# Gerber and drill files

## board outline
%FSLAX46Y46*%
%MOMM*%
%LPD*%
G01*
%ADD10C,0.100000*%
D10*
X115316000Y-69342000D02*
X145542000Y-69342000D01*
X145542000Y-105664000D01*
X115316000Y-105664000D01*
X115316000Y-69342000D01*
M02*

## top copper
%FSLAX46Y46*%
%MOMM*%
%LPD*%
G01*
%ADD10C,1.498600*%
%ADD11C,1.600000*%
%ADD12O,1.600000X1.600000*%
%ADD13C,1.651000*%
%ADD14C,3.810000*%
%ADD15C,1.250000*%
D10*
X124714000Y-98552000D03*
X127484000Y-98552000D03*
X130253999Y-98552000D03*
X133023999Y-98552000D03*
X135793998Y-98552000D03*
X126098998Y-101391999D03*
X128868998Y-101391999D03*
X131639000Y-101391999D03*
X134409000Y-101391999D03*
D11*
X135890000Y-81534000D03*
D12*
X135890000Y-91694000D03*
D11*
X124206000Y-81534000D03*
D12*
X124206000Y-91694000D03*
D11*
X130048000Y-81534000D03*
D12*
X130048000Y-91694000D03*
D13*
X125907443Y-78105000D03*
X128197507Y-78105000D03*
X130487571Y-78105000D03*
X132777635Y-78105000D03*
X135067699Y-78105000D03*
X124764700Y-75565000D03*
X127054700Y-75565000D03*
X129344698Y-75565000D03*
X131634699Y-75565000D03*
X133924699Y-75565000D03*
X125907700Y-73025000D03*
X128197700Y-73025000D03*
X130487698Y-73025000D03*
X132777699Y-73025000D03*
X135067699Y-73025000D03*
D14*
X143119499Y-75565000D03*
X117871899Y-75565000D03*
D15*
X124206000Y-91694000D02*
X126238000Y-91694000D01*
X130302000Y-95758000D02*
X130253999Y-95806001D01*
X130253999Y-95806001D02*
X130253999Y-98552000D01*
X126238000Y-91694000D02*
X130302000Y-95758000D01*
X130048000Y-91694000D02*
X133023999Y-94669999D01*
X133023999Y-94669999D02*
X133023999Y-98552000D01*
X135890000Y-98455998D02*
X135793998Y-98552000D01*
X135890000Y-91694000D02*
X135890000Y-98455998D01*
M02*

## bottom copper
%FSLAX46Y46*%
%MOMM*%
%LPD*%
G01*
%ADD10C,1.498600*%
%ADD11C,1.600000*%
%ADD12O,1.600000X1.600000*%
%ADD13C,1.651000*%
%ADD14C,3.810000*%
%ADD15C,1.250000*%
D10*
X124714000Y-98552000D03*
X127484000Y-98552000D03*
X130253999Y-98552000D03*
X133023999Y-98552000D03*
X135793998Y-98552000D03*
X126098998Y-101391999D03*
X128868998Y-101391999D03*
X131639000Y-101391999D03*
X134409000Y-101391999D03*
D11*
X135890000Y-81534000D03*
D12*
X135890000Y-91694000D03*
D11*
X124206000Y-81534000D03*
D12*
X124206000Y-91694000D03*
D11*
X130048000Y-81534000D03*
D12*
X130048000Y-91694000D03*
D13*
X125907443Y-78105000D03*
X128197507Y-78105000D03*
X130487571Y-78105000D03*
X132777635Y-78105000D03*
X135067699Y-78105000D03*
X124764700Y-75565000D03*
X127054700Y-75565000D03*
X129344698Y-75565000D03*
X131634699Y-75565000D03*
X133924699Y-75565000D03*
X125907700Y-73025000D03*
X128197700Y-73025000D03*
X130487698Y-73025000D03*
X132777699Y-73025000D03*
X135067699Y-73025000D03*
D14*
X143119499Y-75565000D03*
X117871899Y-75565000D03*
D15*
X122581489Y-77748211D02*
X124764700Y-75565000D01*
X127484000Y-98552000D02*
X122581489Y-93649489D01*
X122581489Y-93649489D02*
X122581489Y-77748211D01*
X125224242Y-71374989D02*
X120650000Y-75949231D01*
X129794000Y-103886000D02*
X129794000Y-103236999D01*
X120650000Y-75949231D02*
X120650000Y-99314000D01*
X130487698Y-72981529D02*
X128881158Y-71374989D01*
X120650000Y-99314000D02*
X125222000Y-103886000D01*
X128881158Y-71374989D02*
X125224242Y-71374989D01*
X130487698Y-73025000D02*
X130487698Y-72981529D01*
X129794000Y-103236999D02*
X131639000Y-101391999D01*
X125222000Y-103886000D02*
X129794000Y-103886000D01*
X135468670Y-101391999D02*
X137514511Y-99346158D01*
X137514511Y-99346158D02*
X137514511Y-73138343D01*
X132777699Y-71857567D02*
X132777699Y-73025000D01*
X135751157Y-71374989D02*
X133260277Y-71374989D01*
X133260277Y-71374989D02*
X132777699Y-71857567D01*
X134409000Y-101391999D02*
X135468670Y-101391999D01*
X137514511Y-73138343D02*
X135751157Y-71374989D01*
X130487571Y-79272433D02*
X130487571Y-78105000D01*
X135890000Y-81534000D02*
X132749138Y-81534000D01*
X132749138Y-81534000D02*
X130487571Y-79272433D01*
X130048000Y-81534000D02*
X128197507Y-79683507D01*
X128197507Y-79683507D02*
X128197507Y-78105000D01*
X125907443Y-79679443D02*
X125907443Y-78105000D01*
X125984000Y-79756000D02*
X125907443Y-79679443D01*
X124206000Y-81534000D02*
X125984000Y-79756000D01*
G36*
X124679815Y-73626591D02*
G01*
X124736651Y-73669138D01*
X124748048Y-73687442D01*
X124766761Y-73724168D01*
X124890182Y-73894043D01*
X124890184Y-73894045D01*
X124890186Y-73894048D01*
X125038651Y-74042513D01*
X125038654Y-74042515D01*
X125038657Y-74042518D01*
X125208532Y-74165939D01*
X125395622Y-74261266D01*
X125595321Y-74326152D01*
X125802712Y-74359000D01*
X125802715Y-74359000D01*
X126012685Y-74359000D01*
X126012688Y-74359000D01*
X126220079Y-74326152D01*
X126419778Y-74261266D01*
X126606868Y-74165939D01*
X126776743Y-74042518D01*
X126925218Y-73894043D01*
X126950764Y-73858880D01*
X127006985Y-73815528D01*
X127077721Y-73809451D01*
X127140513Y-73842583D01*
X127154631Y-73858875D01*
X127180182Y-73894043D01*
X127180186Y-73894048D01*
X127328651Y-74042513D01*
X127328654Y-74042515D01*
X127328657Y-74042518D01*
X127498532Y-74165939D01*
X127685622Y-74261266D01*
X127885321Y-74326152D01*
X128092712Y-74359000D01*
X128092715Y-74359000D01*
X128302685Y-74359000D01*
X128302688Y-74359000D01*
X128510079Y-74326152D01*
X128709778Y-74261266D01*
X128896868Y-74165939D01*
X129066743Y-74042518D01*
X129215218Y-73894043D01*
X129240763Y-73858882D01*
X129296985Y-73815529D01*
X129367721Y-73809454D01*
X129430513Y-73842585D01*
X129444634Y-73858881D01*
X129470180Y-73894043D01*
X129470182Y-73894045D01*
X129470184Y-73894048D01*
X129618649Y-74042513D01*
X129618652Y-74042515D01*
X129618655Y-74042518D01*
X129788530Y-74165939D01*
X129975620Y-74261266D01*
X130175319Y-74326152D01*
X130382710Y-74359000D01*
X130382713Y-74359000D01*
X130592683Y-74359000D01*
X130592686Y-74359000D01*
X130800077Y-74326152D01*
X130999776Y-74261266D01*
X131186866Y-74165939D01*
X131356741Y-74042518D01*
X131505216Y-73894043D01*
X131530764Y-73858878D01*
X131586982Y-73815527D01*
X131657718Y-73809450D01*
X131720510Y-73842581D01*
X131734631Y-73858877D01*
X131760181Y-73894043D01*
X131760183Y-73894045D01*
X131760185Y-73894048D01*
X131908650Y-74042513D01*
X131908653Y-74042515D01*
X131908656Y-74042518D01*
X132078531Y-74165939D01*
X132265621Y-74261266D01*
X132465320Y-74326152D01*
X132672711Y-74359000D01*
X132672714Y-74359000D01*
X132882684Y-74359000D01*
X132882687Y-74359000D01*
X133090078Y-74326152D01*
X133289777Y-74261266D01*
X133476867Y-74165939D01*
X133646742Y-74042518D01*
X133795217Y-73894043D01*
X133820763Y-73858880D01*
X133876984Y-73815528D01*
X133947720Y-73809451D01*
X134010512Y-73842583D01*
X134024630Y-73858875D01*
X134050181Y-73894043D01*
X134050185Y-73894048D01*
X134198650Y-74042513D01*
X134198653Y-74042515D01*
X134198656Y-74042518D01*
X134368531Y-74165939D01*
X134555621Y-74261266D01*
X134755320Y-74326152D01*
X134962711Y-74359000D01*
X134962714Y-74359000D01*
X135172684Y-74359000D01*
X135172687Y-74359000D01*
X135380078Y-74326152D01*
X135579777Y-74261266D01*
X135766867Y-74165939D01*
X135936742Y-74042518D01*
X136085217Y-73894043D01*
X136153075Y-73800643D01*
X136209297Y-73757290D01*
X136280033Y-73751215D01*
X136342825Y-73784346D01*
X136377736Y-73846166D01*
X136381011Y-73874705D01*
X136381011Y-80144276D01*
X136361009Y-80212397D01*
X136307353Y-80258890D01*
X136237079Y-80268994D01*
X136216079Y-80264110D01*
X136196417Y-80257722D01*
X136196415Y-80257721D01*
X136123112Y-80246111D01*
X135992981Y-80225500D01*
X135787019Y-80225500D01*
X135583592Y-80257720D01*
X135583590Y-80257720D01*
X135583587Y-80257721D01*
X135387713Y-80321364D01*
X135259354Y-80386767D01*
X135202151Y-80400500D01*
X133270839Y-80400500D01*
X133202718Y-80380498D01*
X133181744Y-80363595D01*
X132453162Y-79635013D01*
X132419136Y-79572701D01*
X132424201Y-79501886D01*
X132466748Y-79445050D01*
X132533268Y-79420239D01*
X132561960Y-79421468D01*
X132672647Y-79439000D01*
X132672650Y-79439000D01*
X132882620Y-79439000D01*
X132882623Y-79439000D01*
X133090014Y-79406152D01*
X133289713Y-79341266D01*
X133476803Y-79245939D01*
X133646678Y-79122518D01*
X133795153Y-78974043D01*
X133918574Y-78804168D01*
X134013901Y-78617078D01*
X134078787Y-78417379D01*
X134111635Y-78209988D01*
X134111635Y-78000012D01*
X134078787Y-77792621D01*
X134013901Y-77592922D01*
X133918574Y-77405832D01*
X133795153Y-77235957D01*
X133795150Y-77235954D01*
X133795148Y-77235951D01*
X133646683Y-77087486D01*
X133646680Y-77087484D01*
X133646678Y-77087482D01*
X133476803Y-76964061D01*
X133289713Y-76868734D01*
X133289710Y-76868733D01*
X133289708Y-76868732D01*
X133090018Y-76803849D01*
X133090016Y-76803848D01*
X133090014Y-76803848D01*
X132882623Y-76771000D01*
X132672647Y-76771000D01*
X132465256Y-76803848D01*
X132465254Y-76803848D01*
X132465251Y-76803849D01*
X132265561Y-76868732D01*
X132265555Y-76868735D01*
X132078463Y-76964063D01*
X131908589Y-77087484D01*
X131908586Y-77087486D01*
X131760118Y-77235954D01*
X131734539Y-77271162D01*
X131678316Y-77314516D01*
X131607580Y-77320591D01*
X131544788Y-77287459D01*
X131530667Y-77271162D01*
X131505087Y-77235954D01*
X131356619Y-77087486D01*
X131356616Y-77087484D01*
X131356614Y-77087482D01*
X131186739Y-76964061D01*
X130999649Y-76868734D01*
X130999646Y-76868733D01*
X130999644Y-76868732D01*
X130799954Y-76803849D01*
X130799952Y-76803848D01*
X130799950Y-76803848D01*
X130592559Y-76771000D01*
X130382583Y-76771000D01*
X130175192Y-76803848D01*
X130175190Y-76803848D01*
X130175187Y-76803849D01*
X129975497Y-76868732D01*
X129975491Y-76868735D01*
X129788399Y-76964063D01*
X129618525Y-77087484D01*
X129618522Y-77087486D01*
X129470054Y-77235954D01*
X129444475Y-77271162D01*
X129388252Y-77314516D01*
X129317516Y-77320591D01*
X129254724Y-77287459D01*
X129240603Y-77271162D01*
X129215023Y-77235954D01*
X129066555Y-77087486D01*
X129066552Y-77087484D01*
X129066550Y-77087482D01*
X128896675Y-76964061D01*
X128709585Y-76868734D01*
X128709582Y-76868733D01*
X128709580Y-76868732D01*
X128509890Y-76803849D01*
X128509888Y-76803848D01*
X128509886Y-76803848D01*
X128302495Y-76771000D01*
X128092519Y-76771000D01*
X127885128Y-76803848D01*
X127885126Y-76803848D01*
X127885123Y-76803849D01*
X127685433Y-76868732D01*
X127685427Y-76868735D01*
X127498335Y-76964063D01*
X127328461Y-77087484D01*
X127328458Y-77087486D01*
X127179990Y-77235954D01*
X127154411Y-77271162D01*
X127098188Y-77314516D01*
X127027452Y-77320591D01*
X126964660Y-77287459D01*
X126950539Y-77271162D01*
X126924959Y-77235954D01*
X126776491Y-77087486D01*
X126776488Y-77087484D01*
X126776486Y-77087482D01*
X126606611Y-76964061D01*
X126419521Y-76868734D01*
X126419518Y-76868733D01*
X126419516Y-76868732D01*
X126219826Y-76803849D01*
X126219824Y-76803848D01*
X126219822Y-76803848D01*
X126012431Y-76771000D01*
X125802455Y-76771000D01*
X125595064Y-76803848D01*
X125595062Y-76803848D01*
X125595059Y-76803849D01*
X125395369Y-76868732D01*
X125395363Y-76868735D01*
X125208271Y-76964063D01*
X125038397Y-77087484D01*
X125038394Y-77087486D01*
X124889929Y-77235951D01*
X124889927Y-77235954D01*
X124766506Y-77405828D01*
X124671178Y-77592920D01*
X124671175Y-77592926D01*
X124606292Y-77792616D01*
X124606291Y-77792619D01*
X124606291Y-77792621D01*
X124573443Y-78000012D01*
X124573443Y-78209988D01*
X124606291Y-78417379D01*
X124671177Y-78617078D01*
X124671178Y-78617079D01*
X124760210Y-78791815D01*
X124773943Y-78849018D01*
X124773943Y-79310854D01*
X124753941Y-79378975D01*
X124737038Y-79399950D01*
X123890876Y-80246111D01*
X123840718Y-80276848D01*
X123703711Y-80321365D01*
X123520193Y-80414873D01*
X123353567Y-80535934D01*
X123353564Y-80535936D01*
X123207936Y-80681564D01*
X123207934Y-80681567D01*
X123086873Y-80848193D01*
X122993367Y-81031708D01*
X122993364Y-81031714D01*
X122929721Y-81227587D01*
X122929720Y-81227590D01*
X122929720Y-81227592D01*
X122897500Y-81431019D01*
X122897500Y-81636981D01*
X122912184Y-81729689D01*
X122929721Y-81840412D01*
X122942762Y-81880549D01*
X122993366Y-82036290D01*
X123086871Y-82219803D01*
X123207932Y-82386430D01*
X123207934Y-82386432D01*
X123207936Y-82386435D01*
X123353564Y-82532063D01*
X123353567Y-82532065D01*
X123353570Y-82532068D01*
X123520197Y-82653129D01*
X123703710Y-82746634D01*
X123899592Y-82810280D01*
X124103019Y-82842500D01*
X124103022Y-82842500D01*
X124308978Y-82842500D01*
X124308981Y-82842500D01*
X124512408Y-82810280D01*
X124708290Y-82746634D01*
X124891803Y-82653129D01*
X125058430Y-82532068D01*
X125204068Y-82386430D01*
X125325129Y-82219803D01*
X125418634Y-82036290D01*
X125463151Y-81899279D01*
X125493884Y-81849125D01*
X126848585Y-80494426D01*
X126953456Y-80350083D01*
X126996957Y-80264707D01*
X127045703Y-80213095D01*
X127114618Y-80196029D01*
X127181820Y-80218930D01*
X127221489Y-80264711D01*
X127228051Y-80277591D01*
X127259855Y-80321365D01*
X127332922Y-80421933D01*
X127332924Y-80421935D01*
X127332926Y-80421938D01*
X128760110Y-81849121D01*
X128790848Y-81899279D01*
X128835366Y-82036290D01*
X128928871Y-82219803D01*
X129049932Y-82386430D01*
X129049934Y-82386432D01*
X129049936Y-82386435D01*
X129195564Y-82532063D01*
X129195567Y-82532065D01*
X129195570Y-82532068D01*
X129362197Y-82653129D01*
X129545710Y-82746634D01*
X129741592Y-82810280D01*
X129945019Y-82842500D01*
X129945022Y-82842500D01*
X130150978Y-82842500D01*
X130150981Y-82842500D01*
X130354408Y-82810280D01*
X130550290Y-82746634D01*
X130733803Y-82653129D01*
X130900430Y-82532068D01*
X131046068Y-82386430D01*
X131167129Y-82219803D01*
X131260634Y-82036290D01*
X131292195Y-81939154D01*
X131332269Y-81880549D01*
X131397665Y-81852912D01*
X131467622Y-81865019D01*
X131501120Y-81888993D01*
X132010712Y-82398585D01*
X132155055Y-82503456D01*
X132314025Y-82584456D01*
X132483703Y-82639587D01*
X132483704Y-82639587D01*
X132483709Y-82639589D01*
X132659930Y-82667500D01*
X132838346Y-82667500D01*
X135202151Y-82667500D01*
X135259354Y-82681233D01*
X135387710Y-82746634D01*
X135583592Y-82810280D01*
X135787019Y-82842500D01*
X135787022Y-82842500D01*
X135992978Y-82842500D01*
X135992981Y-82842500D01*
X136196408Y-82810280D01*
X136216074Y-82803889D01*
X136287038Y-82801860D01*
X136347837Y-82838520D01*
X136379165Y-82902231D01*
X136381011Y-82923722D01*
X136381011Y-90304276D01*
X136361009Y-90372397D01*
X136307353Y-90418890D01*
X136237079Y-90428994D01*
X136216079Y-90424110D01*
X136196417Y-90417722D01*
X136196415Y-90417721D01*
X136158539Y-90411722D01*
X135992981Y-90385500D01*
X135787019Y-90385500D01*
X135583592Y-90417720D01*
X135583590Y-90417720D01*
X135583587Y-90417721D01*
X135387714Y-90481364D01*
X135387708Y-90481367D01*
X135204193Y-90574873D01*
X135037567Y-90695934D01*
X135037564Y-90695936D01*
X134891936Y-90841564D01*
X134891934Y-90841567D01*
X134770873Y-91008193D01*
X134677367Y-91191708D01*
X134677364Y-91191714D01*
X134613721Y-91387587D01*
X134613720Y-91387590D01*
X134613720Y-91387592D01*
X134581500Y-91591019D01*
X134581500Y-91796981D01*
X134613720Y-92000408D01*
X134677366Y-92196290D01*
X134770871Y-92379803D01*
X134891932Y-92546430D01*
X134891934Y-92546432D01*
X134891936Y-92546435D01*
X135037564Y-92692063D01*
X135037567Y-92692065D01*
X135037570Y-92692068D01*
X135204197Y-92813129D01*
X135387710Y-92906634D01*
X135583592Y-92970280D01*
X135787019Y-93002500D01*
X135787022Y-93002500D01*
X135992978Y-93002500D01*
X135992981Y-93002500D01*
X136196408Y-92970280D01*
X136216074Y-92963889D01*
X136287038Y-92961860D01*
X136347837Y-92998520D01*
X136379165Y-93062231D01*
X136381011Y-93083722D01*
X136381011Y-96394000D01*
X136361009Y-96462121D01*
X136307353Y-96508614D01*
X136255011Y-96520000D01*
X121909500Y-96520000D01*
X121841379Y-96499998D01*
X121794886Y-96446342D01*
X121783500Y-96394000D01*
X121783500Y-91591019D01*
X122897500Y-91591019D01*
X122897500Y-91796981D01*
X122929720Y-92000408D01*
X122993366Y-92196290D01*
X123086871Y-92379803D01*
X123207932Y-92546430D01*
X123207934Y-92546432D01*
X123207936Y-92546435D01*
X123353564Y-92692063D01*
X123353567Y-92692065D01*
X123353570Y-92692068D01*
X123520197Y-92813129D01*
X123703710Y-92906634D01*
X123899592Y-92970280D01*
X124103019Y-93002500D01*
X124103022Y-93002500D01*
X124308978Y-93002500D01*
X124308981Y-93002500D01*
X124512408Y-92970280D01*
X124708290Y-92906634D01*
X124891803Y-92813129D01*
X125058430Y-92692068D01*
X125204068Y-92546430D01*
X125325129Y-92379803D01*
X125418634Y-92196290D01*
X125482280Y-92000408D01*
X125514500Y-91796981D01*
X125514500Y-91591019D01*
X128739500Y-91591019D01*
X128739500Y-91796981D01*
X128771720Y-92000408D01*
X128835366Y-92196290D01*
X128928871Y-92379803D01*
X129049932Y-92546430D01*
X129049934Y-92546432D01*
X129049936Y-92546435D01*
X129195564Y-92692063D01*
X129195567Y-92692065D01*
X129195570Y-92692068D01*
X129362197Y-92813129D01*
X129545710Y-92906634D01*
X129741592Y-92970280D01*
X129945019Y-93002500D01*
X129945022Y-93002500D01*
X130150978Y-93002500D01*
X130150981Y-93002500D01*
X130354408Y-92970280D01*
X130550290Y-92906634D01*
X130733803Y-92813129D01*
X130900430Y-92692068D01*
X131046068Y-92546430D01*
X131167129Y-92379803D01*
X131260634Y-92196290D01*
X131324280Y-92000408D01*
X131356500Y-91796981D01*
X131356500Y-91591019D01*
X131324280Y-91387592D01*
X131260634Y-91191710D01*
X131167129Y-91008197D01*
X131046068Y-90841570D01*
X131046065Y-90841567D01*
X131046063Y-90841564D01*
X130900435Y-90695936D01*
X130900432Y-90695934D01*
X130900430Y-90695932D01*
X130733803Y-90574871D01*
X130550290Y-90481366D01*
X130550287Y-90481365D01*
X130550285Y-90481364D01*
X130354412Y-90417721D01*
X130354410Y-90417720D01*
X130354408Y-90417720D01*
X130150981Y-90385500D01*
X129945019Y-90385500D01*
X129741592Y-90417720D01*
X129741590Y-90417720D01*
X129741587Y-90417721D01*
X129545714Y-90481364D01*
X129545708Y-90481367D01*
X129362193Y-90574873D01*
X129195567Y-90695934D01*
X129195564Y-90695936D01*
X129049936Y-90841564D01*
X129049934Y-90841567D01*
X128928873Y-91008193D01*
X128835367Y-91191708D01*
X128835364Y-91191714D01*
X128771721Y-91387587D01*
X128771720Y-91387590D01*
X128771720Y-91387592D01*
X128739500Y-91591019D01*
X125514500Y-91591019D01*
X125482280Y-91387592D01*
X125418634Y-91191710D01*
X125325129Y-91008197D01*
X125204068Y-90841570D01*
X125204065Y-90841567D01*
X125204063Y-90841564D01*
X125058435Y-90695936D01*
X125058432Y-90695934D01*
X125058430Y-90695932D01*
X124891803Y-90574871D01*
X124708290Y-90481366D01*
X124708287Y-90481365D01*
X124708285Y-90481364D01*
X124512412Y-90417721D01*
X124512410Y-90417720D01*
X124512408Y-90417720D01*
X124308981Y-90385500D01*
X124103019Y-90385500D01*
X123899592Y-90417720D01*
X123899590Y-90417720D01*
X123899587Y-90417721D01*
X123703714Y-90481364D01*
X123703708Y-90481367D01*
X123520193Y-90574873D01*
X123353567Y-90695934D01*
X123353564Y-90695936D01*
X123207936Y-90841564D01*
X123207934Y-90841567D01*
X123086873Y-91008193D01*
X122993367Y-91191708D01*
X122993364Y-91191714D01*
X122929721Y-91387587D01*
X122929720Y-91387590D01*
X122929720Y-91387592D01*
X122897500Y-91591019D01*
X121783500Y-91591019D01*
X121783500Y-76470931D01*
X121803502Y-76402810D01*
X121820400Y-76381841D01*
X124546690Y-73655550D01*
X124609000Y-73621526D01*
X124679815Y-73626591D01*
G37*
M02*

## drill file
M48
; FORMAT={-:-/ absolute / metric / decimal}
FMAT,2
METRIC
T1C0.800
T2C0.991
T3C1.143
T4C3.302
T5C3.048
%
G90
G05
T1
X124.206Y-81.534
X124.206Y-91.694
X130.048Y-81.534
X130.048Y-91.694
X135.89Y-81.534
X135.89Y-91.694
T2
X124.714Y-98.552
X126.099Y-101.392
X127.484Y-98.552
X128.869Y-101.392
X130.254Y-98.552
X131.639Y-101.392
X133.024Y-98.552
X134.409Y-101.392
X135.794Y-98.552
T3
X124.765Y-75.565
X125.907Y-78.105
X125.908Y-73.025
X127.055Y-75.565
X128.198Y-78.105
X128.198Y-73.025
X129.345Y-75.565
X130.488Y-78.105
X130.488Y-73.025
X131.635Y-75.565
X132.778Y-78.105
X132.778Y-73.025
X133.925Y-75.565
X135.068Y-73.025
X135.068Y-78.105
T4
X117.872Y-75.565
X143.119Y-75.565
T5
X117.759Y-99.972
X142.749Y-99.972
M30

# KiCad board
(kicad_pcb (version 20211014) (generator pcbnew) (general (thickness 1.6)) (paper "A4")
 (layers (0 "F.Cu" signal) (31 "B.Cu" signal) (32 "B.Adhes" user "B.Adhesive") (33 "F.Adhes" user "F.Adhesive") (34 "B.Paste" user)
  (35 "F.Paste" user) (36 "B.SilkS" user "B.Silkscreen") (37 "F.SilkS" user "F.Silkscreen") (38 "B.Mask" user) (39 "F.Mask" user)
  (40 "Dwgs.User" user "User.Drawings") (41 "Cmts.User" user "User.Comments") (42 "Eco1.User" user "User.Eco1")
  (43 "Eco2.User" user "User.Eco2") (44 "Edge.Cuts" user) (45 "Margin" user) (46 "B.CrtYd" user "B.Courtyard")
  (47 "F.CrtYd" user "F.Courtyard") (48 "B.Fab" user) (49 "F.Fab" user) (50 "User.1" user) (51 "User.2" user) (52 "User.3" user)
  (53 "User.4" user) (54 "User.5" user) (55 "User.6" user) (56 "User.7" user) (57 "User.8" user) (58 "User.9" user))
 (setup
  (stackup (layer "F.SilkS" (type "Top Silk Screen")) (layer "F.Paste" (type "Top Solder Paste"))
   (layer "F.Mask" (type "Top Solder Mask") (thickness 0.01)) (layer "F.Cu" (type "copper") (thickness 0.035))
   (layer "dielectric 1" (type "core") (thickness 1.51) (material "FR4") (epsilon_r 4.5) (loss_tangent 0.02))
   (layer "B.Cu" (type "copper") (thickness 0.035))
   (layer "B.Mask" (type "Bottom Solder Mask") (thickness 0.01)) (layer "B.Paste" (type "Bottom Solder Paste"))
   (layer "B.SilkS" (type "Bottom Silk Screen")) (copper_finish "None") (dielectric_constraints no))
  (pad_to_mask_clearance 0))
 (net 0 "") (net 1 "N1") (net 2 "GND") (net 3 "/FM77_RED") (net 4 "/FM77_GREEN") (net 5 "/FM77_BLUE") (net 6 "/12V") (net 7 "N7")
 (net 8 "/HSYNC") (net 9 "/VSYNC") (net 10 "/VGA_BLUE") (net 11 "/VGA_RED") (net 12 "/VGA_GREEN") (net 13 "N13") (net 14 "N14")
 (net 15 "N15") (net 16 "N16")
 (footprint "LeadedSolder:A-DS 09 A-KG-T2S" (layer "F.Cu") (at 124.714 98.552)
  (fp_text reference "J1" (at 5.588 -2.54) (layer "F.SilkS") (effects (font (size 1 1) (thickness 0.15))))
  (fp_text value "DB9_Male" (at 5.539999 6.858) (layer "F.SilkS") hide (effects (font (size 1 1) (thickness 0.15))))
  (pad "" np_thru_hole circle (at 18.034998 1.419885) (size 3.048 3.048) (drill 3.048) (layers *.Cu *.Mask))
  (pad "" np_thru_hole circle (at -6.955 1.419885) (size 3.048 3.048) (drill 3.048) (layers *.Cu *.Mask))
  (pad "1" thru_hole circle (at 0 0) (size 1.4986 1.4986) (drill 0.9906) (layers *.Cu *.Mask) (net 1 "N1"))
  (pad "2" thru_hole circle (at 2.77 0) (size 1.4986 1.4986) (drill 0.9906) (layers *.Cu *.Mask) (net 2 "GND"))
  (pad "3" thru_hole circle (at 5.539999 0) (size 1.4986 1.4986) (drill 0.9906) (layers *.Cu *.Mask) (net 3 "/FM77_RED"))
  (pad "4" thru_hole circle (at 8.309999 0) (size 1.4986 1.4986) (drill 0.9906) (layers *.Cu *.Mask) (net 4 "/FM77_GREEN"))
  (pad "5" thru_hole circle (at 11.079998 0) (size 1.4986 1.4986) (drill 0.9906) (layers *.Cu *.Mask) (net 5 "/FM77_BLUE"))
  (pad "6" thru_hole circle (at 1.384998 2.839999) (size 1.4986 1.4986) (drill 0.9906) (layers *.Cu *.Mask) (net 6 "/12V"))
  (pad "7" thru_hole circle (at 4.154998 2.839999) (size 1.4986 1.4986) (drill 0.9906) (layers *.Cu *.Mask) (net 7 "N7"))
  (pad "8" thru_hole circle (at 6.925 2.839999) (size 1.4986 1.4986) (drill 0.9906) (layers *.Cu *.Mask) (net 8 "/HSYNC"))
  (pad "9" thru_hole circle (at 9.695 2.839999) (size 1.4986 1.4986) (drill 0.9906) (layers *.Cu *.Mask) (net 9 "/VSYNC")))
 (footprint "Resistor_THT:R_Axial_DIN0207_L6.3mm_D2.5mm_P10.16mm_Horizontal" (layer "F.Cu") (at 135.89 81.534 -90)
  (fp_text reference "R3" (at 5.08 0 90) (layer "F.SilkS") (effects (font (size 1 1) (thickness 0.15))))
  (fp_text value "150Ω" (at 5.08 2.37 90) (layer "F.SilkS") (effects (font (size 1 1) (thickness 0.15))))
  (pad "1" thru_hole circle (at 0 0 270) (size 1.6 1.6) (drill 0.8) (layers *.Cu *.Mask) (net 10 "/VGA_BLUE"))
  (pad "2" thru_hole oval (at 10.16 0 270) (size 1.6 1.6) (drill 0.8) (layers *.Cu *.Mask) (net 5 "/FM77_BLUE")))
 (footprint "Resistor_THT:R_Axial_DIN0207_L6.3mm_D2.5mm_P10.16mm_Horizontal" (layer "F.Cu") (at 124.206 81.534 -90)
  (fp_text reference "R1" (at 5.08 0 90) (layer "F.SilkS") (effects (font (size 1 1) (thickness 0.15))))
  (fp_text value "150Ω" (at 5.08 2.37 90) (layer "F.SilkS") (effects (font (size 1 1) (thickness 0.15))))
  (pad "1" thru_hole circle (at 0 0 270) (size 1.6 1.6) (drill 0.8) (layers *.Cu *.Mask) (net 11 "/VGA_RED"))
  (pad "2" thru_hole oval (at 10.16 0 270) (size 1.6 1.6) (drill 0.8) (layers *.Cu *.Mask) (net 3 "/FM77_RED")))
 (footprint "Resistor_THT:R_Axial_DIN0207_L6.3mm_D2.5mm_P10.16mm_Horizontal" (layer "F.Cu") (at 130.048 81.534 -90)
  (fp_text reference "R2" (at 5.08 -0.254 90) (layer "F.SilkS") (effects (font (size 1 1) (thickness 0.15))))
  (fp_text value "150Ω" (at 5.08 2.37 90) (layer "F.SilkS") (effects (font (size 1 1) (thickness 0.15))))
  (pad "1" thru_hole circle (at 0 0 270) (size 1.6 1.6) (drill 0.8) (layers *.Cu *.Mask) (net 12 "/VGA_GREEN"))
  (pad "2" thru_hole oval (at 10.16 0 270) (size 1.6 1.6) (drill 0.8) (layers *.Cu *.Mask) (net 4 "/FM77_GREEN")))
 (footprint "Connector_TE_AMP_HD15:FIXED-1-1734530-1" (layer "F.Cu") (at 130.495699 63.754)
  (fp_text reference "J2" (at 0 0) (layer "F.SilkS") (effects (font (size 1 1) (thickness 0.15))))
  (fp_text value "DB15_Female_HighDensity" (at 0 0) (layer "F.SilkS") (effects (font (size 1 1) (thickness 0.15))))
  (pad "1" thru_hole circle locked (at -4.588256 14.351) (size 1.651 1.651) (drill 1.143) (layers *.Cu *.Mask) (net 11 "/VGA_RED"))
  (pad "2" thru_hole circle locked (at -2.298192 14.351) (size 1.651 1.651) (drill 1.143) (layers *.Cu *.Mask) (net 12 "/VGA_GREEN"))
  (pad "3" thru_hole circle locked (at -0.008128 14.351) (size 1.651 1.651) (drill 1.143) (layers *.Cu *.Mask) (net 10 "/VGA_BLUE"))
  (pad "4" thru_hole circle locked (at 2.281936 14.351) (size 1.651 1.651) (drill 1.143) (layers *.Cu *.Mask) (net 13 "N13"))
  (pad "5" thru_hole circle locked (at 4.572 14.351) (size 1.651 1.651) (drill 1.143) (layers *.Cu *.Mask) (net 2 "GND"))
  (pad "6" thru_hole circle locked (at -5.730999 11.811) (size 1.651 1.651) (drill 1.143) (layers *.Cu *.Mask) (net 2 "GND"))
  (pad "7" thru_hole circle locked (at -3.440999 11.811) (size 1.651 1.651) (drill 1.143) (layers *.Cu *.Mask) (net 2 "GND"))
  (pad "8" thru_hole circle locked (at -1.151001 11.811) (size 1.651 1.651) (drill 1.143) (layers *.Cu *.Mask) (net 2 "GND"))
  (pad "9" thru_hole circle locked (at 1.139 11.811) (size 1.651 1.651) (drill 1.143) (layers *.Cu *.Mask) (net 2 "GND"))
  (pad "10" thru_hole circle locked (at 3.429 11.811) (size 1.651 1.651) (drill 1.143) (layers *.Cu *.Mask) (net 2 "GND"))
  (pad "11" thru_hole circle locked (at -4.587999 9.271) (size 1.651 1.651) (drill 1.143) (layers *.Cu *.Mask) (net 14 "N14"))
  (pad "12" thru_hole circle locked (at -2.297999 9.271) (size 1.651 1.651) (drill 1.143) (layers *.Cu *.Mask) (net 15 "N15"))
  (pad "13" thru_hole circle locked (at -0.008001 9.271) (size 1.651 1.651) (drill 1.143) (layers *.Cu *.Mask) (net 8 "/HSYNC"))
  (pad "14" thru_hole circle locked (at 2.282 9.271) (size 1.651 1.651) (drill 1.143) (layers *.Cu *.Mask) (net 9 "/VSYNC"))
  (pad "15" thru_hole circle locked (at 4.572 9.271) (size 1.651 1.651) (drill 1.143) (layers *.Cu *.Mask) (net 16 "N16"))
  (pad "16" thru_hole circle locked (at 12.6238 11.811) (size 3.81 3.81) (drill 3.302) (layers *.Cu *.Mask))
  (pad "17" thru_hole circle locked (at -12.6238 11.811) (size 3.81 3.81) (drill 3.302) (layers *.Cu *.Mask)))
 (gr_rect (start 115.316 105.664) (end 145.542 69.342) (layer "Edge.Cuts") (width 0.1) (fill none))
 (segment (start 122.581489 77.748211) (end 124.7647 75.565) (width 1.25) (layer "B.Cu") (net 2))
 (segment (start 127.484 98.552) (end 122.581489 93.649489) (width 1.25) (layer "B.Cu") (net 2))
 (segment (start 122.581489 93.649489) (end 122.581489 77.748211) (width 1.25) (layer "B.Cu") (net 2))
 (segment (start 124.206 91.694) (end 126.238 91.694) (width 1.25) (layer "F.Cu") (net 3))
 (segment (start 130.302 95.758) (end 130.253999 95.806001) (width 1.25) (layer "F.Cu") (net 3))
 (segment (start 130.253999 95.806001) (end 130.253999 98.552) (width 1.25) (layer "F.Cu") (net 3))
 (segment (start 126.238 91.694) (end 130.302 95.758) (width 1.25) (layer "F.Cu") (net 3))
 (segment (start 130.048 91.694) (end 133.023999 94.669999) (width 1.25) (layer "F.Cu") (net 4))
 (segment (start 133.023999 94.669999) (end 133.023999 98.552) (width 1.25) (layer "F.Cu") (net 4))
 (segment (start 135.89 98.455998) (end 135.793998 98.552) (width 1.25) (layer "F.Cu") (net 5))
 (segment (start 135.89 91.694) (end 135.89 98.455998) (width 1.25) (layer "F.Cu") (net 5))
 (segment (start 125.224242 71.374989) (end 120.65 75.949231) (width 1.25) (layer "B.Cu") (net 8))
 (segment (start 129.794 103.886) (end 129.794 103.236999) (width 1.25) (layer "B.Cu") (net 8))
 (segment (start 120.65 75.949231) (end 120.65 99.314) (width 1.25) (layer "B.Cu") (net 8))
 (segment (start 130.487698 72.981529) (end 128.881158 71.374989) (width 1.25) (layer "B.Cu") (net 8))
 (segment (start 120.65 99.314) (end 125.222 103.886) (width 1.25) (layer "B.Cu") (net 8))
 (segment (start 128.881158 71.374989) (end 125.224242 71.374989) (width 1.25) (layer "B.Cu") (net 8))
 (segment (start 130.487698 73.025) (end 130.487698 72.981529) (width 1.25) (layer "B.Cu") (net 8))
 (segment (start 129.794 103.236999) (end 131.639 101.391999) (width 1.25) (layer "B.Cu") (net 8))
 (segment (start 125.222 103.886) (end 129.794 103.886) (width 1.25) (layer "B.Cu") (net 8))
 (segment (start 135.46867 101.391999) (end 137.514511 99.346158) (width 1.25) (layer "B.Cu") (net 9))
 (segment (start 137.514511 99.346158) (end 137.514511 73.138343) (width 1.25) (layer "B.Cu") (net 9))
 (segment (start 132.777699 71.857567) (end 132.777699 73.025) (width 1.25) (layer "B.Cu") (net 9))
 (segment (start 135.751157 71.374989) (end 133.260277 71.374989) (width 1.25) (layer "B.Cu") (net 9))
 (segment (start 133.260277 71.374989) (end 132.777699 71.857567) (width 1.25) (layer "B.Cu") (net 9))
 (segment (start 134.409 101.391999) (end 135.46867 101.391999) (width 1.25) (layer "B.Cu") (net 9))
 (segment (start 137.514511 73.138343) (end 135.751157 71.374989) (width 1.25) (layer "B.Cu") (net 9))
 (segment (start 130.487571 79.272433) (end 130.487571 78.105) (width 1.25) (layer "B.Cu") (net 10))
 (segment (start 135.89 81.534) (end 132.749138 81.534) (width 1.25) (layer "B.Cu") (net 10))
 (segment (start 132.749138 81.534) (end 130.487571 79.272433) (width 1.25) (layer "B.Cu") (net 10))
 (segment (start 130.048 81.534) (end 128.197507 79.683507) (width 1.25) (layer "B.Cu") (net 12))
 (segment (start 128.197507 79.683507) (end 128.197507 78.105) (width 1.25) (layer "B.Cu") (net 12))
 (segment (start 125.907443 79.679443) (end 125.907443 78.105) (width 1.25) (layer "B.Cu") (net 11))
 (segment (start 125.984 79.756) (end 125.907443 79.679443) (width 1.25) (layer "B.Cu") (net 11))
 (segment (start 124.206 81.534) (end 125.984 79.756) (width 1.25) (layer "B.Cu") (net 11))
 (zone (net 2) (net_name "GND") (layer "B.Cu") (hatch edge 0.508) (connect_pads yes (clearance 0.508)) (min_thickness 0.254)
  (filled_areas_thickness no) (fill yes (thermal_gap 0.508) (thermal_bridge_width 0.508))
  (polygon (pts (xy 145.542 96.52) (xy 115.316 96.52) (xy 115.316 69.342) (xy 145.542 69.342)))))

